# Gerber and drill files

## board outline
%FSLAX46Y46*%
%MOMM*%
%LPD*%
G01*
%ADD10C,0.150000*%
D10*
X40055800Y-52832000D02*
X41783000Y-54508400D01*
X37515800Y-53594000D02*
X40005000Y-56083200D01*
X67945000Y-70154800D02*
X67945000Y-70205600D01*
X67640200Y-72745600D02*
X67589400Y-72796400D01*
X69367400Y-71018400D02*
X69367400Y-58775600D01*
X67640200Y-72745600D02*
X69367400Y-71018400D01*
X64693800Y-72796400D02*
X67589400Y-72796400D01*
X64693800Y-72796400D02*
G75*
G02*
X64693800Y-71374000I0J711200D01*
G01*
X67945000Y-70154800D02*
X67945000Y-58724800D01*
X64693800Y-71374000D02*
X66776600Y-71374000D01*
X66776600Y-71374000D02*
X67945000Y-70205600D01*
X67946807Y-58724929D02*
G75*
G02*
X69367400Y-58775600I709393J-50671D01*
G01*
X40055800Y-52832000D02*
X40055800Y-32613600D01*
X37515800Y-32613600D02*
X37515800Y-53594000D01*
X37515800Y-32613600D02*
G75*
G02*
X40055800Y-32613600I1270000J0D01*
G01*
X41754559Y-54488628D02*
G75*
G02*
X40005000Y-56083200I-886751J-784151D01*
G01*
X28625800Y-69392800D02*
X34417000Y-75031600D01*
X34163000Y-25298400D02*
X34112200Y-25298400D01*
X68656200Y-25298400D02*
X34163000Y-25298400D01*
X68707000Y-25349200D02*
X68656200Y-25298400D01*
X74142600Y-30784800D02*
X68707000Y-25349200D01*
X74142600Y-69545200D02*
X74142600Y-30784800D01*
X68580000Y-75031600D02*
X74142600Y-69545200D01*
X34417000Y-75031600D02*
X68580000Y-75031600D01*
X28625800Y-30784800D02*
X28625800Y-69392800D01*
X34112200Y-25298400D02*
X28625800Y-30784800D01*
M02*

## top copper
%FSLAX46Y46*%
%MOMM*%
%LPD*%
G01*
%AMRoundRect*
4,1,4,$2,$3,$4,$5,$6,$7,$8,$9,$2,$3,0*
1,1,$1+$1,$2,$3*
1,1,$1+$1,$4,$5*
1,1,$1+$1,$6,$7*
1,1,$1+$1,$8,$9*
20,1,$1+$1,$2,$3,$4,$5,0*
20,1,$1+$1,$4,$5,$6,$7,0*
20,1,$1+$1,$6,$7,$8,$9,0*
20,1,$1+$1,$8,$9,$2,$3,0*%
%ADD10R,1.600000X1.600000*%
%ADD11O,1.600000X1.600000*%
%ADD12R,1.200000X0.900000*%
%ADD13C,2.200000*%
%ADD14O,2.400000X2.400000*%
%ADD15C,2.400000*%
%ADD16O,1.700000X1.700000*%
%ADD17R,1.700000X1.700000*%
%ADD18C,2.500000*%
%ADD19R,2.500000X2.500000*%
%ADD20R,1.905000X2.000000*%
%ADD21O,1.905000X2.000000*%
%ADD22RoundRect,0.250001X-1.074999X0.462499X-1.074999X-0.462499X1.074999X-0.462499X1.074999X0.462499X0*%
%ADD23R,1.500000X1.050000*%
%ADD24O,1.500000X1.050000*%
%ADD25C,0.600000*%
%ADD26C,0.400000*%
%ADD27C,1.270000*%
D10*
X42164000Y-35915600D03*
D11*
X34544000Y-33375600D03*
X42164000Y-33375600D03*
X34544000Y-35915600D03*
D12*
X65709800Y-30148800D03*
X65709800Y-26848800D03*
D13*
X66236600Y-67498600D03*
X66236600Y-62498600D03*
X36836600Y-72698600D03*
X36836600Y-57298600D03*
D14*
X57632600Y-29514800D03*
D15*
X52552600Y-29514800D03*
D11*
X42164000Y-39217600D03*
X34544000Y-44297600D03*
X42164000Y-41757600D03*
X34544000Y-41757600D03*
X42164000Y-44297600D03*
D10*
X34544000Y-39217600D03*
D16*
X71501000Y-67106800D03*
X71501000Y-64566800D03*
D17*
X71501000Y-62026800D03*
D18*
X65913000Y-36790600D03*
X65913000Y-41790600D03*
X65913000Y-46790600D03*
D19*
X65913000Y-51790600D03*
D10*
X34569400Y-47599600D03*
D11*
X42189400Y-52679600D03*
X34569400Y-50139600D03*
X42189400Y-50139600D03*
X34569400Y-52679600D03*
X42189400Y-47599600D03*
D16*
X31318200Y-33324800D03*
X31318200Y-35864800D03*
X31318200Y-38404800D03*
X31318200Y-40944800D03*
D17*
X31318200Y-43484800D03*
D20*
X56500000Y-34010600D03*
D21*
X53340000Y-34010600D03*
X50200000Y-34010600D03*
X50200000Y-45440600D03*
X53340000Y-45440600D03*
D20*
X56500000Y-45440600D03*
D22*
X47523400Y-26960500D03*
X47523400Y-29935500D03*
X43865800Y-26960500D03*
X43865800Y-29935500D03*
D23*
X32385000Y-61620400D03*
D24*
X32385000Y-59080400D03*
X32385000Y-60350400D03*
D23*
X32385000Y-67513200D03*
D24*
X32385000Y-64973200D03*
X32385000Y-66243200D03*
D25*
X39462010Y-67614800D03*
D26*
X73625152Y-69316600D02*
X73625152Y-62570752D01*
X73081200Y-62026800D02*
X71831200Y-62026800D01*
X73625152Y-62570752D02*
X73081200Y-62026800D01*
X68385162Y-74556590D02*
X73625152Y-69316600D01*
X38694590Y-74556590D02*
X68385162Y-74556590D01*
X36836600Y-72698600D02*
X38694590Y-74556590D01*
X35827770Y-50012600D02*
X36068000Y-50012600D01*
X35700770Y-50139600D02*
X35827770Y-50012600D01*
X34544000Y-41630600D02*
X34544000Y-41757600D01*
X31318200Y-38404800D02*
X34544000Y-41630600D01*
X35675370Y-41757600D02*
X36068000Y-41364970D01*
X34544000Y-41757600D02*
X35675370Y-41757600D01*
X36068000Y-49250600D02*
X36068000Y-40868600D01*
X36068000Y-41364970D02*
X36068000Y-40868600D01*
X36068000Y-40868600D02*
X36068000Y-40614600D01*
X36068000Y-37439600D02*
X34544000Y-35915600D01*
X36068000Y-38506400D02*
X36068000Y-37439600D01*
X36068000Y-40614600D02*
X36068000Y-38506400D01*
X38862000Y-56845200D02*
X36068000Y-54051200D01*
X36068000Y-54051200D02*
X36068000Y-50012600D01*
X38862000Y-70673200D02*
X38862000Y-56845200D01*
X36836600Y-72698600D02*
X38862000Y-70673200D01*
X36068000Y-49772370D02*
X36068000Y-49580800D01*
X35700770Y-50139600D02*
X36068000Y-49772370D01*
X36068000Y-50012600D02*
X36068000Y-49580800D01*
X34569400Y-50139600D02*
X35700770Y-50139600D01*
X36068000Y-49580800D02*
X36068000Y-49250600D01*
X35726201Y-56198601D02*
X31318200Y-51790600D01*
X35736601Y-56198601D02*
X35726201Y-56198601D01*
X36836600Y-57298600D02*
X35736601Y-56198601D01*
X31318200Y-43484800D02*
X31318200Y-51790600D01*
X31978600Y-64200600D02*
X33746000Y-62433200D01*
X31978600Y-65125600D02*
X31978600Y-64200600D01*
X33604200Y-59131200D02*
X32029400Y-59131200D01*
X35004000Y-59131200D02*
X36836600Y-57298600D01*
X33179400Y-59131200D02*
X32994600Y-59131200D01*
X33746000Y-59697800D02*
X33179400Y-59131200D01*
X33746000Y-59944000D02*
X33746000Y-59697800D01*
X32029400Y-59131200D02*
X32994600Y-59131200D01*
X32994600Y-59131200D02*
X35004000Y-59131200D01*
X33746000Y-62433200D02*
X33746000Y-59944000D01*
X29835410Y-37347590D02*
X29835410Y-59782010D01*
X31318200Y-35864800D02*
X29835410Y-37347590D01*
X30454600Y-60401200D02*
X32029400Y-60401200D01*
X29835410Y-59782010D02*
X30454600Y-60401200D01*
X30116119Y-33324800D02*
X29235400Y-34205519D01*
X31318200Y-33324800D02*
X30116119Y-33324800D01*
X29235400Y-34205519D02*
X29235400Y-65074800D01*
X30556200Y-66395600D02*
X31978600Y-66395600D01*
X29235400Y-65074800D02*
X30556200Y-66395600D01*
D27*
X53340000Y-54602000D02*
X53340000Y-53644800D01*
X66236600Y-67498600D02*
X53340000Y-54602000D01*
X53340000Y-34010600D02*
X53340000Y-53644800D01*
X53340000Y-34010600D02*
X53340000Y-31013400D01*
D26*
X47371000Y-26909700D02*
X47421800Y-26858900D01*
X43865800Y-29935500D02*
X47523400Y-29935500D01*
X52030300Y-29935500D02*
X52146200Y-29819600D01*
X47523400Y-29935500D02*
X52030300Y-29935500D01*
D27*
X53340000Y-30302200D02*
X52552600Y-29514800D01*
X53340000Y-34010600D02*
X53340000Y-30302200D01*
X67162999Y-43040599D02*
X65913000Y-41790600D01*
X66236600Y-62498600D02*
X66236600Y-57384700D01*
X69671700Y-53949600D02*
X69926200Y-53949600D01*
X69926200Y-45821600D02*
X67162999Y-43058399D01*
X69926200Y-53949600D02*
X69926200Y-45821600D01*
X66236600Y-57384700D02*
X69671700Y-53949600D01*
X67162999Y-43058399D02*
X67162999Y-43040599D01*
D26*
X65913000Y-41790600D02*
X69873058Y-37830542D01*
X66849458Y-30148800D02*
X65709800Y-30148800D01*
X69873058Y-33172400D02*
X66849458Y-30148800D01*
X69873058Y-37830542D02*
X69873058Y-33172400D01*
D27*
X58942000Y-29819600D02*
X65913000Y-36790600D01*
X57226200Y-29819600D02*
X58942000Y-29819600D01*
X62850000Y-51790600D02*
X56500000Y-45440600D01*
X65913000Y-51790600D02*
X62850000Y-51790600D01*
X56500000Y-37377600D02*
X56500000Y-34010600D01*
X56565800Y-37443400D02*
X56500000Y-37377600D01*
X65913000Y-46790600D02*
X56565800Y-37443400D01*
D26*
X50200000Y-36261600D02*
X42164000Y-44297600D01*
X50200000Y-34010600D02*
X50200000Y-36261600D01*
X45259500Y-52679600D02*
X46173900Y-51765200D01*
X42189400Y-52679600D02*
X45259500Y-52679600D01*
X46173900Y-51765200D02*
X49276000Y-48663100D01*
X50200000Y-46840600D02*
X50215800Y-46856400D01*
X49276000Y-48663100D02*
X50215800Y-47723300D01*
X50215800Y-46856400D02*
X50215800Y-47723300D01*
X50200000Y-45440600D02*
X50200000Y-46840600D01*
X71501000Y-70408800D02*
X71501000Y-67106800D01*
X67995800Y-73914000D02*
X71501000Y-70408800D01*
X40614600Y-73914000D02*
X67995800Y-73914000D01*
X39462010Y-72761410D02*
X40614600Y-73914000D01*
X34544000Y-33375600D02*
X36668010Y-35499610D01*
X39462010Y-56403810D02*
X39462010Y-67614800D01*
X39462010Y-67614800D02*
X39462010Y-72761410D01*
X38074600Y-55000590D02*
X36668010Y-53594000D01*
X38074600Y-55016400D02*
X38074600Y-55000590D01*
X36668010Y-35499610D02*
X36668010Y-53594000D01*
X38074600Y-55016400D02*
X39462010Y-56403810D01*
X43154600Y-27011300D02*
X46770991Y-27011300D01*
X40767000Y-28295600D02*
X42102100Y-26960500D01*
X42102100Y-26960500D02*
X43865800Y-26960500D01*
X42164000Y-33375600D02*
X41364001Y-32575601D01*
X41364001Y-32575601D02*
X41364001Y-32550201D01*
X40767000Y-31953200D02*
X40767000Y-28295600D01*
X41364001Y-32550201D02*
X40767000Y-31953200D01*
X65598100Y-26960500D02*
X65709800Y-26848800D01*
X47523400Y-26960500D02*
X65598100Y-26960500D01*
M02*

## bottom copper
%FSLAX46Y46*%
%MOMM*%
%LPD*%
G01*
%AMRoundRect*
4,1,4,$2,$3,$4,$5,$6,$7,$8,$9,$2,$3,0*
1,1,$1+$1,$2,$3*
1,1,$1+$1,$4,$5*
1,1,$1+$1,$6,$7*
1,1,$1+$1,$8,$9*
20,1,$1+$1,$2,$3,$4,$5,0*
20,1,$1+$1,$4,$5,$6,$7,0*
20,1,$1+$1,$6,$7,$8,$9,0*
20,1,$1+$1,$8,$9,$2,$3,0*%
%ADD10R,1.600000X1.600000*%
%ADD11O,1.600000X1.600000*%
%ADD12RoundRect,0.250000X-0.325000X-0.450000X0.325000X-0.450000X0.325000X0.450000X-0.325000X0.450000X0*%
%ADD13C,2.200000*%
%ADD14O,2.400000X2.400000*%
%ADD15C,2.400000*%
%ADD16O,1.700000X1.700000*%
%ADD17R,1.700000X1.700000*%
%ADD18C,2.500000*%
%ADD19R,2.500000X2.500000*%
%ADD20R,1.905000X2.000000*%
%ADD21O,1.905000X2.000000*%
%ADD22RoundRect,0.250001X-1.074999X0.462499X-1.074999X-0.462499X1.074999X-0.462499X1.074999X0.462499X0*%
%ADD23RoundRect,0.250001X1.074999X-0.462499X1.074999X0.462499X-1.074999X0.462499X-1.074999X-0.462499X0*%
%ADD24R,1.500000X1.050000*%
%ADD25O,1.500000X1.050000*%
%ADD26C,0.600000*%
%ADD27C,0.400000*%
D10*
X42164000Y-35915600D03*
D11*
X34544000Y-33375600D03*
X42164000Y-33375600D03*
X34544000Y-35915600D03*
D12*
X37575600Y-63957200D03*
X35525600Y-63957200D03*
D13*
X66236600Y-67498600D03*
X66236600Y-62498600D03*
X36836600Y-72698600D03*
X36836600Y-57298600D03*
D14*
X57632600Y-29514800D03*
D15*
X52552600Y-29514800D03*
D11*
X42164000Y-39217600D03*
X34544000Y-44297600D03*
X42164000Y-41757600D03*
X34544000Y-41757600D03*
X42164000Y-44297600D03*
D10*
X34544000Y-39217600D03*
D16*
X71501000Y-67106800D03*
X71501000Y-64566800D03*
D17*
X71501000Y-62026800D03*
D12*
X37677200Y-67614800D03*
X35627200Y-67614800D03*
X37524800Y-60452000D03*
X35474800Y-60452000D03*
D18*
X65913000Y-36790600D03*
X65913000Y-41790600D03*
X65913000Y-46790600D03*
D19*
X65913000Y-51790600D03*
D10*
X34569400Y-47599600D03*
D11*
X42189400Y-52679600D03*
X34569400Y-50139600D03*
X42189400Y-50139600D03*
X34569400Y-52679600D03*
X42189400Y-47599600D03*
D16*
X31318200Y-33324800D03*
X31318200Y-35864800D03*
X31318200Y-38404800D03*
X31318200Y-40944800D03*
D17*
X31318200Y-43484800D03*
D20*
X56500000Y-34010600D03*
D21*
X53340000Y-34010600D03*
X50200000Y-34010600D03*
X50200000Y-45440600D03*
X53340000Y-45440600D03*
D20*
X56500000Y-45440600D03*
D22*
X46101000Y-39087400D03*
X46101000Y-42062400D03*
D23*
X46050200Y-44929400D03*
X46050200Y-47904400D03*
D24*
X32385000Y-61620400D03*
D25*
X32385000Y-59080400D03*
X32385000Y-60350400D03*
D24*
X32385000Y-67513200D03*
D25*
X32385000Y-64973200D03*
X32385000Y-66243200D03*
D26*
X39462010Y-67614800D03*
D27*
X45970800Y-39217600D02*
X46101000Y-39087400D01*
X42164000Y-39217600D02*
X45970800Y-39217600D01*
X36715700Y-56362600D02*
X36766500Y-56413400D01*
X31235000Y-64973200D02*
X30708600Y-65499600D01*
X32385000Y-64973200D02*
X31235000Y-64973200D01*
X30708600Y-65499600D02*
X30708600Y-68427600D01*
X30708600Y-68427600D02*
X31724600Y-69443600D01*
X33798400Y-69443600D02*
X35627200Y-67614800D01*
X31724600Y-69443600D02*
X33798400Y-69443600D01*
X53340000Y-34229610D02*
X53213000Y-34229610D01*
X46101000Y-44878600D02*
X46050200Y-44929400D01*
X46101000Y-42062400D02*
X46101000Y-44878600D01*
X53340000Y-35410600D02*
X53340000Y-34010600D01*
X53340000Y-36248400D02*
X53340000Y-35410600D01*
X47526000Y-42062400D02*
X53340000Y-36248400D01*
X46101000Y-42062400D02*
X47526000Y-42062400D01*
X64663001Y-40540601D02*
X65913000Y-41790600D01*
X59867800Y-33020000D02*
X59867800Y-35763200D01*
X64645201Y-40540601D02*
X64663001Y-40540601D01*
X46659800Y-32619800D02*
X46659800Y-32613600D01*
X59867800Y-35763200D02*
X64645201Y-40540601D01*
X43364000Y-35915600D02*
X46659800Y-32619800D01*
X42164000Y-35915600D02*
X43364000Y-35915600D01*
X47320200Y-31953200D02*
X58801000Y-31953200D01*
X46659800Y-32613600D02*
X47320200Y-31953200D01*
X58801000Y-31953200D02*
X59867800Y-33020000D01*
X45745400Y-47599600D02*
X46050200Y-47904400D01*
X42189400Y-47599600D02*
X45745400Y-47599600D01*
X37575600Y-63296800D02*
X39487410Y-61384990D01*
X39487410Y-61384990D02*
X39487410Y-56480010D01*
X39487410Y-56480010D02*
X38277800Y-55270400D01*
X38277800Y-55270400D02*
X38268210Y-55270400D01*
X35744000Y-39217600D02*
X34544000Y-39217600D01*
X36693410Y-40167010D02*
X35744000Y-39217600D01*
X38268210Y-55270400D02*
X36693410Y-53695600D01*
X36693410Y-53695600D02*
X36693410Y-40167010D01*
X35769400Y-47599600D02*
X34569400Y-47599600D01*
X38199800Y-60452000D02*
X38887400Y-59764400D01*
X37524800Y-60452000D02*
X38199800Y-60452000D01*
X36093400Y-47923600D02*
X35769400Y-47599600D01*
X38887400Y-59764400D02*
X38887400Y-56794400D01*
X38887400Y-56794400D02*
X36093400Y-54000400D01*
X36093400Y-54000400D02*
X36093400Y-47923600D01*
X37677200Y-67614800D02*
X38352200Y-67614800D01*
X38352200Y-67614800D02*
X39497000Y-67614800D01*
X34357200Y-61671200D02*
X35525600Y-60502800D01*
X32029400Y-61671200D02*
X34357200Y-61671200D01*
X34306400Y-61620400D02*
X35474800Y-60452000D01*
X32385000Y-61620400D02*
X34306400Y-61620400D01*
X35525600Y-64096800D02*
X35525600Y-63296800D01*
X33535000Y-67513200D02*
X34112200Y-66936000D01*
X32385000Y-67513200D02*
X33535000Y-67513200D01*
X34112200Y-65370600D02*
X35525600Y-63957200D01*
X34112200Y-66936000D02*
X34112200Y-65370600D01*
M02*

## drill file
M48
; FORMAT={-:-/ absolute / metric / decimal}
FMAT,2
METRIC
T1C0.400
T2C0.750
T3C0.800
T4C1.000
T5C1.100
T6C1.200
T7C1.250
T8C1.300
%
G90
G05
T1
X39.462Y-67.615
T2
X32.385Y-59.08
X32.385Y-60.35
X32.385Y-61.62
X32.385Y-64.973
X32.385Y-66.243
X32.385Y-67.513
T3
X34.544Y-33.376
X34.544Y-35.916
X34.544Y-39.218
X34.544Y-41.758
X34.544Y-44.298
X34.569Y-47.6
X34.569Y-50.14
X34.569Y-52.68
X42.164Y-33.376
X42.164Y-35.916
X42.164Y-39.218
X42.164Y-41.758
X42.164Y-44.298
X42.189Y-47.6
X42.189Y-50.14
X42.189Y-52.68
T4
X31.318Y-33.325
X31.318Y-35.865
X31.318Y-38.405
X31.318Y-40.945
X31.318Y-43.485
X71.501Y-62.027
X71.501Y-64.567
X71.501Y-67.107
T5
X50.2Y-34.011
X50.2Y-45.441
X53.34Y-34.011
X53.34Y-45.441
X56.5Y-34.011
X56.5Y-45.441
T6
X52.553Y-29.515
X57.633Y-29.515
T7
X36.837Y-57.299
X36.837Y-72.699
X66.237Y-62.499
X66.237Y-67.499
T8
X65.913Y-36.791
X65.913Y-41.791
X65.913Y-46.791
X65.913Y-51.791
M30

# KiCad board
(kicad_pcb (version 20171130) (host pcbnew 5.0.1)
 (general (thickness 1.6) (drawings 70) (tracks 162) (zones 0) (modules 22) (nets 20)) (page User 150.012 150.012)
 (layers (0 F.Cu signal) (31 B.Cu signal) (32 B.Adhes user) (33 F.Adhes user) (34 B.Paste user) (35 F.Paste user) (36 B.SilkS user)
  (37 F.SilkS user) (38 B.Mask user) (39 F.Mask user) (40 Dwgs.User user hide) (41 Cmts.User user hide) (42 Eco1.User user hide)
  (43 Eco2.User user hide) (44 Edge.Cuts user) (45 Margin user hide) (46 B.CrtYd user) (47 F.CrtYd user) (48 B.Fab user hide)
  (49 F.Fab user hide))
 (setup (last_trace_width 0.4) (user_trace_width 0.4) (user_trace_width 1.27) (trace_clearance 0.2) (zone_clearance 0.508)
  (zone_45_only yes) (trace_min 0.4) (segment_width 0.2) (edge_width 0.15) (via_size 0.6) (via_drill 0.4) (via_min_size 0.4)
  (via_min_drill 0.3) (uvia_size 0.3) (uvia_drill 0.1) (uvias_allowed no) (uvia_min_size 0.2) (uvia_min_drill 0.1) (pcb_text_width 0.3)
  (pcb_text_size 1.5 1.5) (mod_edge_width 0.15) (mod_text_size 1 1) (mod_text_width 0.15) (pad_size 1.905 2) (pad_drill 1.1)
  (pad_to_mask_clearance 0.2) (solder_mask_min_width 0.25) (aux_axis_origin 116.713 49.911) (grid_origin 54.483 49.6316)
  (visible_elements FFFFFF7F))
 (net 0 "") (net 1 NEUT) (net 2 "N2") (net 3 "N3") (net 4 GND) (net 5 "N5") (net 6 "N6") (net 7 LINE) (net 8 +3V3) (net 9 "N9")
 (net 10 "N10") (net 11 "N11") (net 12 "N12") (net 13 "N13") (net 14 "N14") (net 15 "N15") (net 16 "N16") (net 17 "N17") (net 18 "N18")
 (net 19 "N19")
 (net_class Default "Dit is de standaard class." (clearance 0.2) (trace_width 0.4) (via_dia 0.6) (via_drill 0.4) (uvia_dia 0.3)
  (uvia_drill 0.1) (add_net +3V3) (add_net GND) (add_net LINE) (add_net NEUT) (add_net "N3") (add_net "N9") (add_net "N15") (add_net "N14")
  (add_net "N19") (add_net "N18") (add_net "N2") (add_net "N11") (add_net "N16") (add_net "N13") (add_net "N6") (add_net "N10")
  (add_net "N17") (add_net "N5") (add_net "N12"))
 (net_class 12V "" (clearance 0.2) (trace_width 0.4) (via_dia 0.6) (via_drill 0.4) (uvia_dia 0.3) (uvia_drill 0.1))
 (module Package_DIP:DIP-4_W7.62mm (layer F.Cu) (at 42.164 35.9156 180)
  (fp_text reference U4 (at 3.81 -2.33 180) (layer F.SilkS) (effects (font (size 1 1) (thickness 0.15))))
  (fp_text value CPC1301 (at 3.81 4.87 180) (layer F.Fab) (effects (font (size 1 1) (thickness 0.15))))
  (pad 1 thru_hole rect (at 0 0 180) (size 1.6 1.6) (drill 0.8) (layers *.Cu *.Mask) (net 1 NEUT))
  (pad 3 thru_hole oval (at 7.62 2.54 180) (size 1.6 1.6) (drill 0.8) (layers *.Cu *.Mask) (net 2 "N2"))
  (pad 2 thru_hole oval (at 0 2.54 180) (size 1.6 1.6) (drill 0.8) (layers *.Cu *.Mask) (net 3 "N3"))
  (pad 4 thru_hole oval (at 7.62 0 180) (size 1.6 1.6) (drill 0.8) (layers *.Cu *.Mask) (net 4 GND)))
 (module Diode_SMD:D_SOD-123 (layer F.Cu) (at 65.7098 28.4988 270)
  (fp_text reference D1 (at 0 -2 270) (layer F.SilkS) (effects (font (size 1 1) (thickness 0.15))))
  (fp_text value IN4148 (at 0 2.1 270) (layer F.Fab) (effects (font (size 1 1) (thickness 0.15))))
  (pad 2 smd rect (at 1.65 0 270) (size 0.9 1.2) (layers F.Cu F.Paste F.Mask) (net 1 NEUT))
  (pad 1 smd rect (at -1.65 0 270) (size 0.9 1.2) (layers F.Cu F.Paste F.Mask) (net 3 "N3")))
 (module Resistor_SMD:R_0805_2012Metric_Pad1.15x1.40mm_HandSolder (layer B.Cu) (at 36.5506 63.9572)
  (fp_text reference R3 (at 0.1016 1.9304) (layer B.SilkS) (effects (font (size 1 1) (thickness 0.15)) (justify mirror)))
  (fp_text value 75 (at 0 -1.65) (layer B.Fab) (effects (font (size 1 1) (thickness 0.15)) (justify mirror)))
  (pad 2 smd roundrect (at 1.025 0) (size 1.15 1.4) (layers B.Cu B.Paste B.Mask) (roundrect_rratio 0.217391) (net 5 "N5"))
  (pad 1 smd roundrect (at -1.025 0) (size 1.15 1.4) (layers B.Cu B.Paste B.Mask) (roundrect_rratio 0.217391) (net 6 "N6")))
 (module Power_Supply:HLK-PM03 (layer F.Cu) (at 51.5366 64.9986 180)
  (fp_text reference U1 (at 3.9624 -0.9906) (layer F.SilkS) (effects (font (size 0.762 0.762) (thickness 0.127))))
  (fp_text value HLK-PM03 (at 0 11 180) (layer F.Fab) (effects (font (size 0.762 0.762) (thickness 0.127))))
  (pad 1 thru_hole circle (at -14.7 -2.5 180) (size 2.2 2.2) (drill 1.25) (layers *.Cu *.Mask) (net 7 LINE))
  (pad 2 thru_hole circle (at -14.7 2.5 180) (size 2.2 2.2) (drill 1.25) (layers *.Cu *.Mask) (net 1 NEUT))
  (pad 3 thru_hole circle (at 14.7 -7.7 180) (size 2.2 2.2) (drill 1.25) (layers *.Cu *.Mask) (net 4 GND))
  (pad 4 thru_hole circle (at 14.7 7.7 180) (size 2.2 2.2) (drill 1.25) (layers *.Cu *.Mask) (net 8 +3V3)))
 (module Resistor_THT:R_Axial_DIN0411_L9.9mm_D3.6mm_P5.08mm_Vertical (layer F.Cu) (at 52.5526 29.5148)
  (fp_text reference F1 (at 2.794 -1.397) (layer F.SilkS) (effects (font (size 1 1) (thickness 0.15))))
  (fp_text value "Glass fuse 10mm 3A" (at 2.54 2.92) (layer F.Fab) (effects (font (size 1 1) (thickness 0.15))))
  (pad 2 thru_hole oval (at 5.08 0) (size 2.4 2.4) (drill 1.2) (layers *.Cu *.Mask) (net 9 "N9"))
  (pad 1 thru_hole circle (at 0 0) (size 2.4 2.4) (drill 1.2) (layers *.Cu *.Mask) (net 7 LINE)))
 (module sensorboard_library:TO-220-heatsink (layer F.Cu) (at 53.3146 37.9476)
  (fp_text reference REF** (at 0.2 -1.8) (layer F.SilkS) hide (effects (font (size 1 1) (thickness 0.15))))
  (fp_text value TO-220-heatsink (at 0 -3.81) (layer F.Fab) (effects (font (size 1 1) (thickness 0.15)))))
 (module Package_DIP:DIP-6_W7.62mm (layer F.Cu) (at 34.544 39.2176)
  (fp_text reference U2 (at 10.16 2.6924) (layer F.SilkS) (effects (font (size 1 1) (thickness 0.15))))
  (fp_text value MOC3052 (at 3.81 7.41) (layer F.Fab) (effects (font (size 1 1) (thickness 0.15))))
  (pad 6 thru_hole oval (at 7.62 0) (size 1.6 1.6) (drill 0.8) (layers *.Cu *.Mask) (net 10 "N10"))
  (pad 3 thru_hole oval (at 0 5.08) (size 1.6 1.6) (drill 0.8) (layers *.Cu *.Mask))
  (pad 5 thru_hole oval (at 7.62 2.54) (size 1.6 1.6) (drill 0.8) (layers *.Cu *.Mask))
  (pad 2 thru_hole oval (at 0 2.54) (size 1.6 1.6) (drill 0.8) (layers *.Cu *.Mask) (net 4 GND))
  (pad 4 thru_hole oval (at 7.62 5.08) (size 1.6 1.6) (drill 0.8) (layers *.Cu *.Mask) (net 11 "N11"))
  (pad 1 thru_hole rect (at 0 0) (size 1.6 1.6) (drill 0.8) (layers *.Cu *.Mask) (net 5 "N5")))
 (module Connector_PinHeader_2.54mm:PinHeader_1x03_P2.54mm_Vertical (layer B.Cu) (at 71.501 62.0268 180)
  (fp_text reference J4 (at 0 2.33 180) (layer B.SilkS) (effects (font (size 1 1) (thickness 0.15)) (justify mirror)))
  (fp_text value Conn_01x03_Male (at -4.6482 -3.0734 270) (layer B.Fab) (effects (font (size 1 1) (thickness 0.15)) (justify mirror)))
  (pad 3 thru_hole oval (at 0 -5.08 180) (size 1.7 1.7) (drill 1) (layers *.Cu *.Mask) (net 2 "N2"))
  (pad 2 thru_hole oval (at 0 -2.54 180) (size 1.7 1.7) (drill 1) (layers *.Cu *.Mask))
  (pad 1 thru_hole rect (at 0 0 180) (size 1.7 1.7) (drill 1) (layers *.Cu *.Mask) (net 4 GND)))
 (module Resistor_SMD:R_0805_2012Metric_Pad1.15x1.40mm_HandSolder (layer B.Cu) (at 36.6522 67.6148)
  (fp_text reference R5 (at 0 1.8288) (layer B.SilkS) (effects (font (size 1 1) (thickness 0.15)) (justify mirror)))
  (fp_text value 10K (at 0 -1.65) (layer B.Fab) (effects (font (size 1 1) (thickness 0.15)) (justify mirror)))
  (pad 2 smd roundrect (at 1.025 0) (size 1.15 1.4) (layers B.Cu B.Paste B.Mask) (roundrect_rratio 0.217391) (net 2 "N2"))
  (pad 1 smd roundrect (at -1.025 0) (size 1.15 1.4) (layers B.Cu B.Paste B.Mask) (roundrect_rratio 0.217391) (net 8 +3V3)))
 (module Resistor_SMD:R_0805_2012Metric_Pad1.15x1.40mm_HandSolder (layer B.Cu) (at 36.4998 60.452)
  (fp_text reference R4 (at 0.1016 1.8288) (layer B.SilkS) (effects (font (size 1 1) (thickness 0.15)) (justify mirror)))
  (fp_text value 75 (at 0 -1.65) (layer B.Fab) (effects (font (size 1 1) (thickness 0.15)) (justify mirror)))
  (pad 2 smd roundrect (at 1.025 0) (size 1.15 1.4) (layers B.Cu B.Paste B.Mask) (roundrect_rratio 0.217391) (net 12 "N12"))
  (pad 1 smd roundrect (at -1.025 0) (size 1.15 1.4) (layers B.Cu B.Paste B.Mask) (roundrect_rratio 0.217391) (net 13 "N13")))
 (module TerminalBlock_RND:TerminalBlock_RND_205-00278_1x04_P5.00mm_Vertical (layer F.Cu) (at 65.913 51.7906 90)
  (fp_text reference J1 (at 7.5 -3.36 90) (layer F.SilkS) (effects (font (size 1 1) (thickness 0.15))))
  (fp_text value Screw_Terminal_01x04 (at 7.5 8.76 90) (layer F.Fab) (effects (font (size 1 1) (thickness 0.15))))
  (pad 4 thru_hole circle (at 15 0 90) (size 2.5 2.5) (drill 1.3) (layers *.Cu *.Mask) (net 9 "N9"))
  (pad 3 thru_hole circle (at 10 0 90) (size 2.5 2.5) (drill 1.3) (layers *.Cu *.Mask) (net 1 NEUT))
  (pad 2 thru_hole circle (at 5 0 90) (size 2.5 2.5) (drill 1.3) (layers *.Cu *.Mask) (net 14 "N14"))
  (pad 1 thru_hole rect (at 0 0 90) (size 2.5 2.5) (drill 1.3) (layers *.Cu *.Mask) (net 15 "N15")))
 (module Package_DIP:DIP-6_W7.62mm (layer F.Cu) (at 34.5694 47.5996)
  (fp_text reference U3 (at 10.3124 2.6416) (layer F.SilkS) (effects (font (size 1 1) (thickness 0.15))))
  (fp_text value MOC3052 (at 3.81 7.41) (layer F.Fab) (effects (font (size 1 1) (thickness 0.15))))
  (pad 1 thru_hole rect (at 0 0) (size 1.6 1.6) (drill 0.8) (layers *.Cu *.Mask) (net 12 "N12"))
  (pad 4 thru_hole oval (at 7.62 5.08) (size 1.6 1.6) (drill 0.8) (layers *.Cu *.Mask) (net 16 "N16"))
  (pad 2 thru_hole oval (at 0 2.54) (size 1.6 1.6) (drill 0.8) (layers *.Cu *.Mask) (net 4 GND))
  (pad 5 thru_hole oval (at 7.62 2.54) (size 1.6 1.6) (drill 0.8) (layers *.Cu *.Mask))
  (pad 3 thru_hole oval (at 0 5.08) (size 1.6 1.6) (drill 0.8) (layers *.Cu *.Mask))
  (pad 6 thru_hole oval (at 7.62 0) (size 1.6 1.6) (drill 0.8) (layers *.Cu *.Mask) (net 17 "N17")))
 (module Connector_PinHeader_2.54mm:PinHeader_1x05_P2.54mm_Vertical (layer B.Cu) (at 31.3182 43.4848)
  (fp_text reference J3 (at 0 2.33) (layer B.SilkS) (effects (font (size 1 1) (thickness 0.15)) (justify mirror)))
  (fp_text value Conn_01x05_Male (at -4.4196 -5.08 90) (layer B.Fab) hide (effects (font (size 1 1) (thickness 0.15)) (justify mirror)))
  (pad 5 thru_hole oval (at 0 -10.16) (size 1.7 1.7) (drill 1) (layers *.Cu *.Mask) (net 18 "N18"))
  (pad 4 thru_hole oval (at 0 -7.62) (size 1.7 1.7) (drill 1) (layers *.Cu *.Mask) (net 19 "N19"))
  (pad 3 thru_hole oval (at 0 -5.08) (size 1.7 1.7) (drill 1) (layers *.Cu *.Mask) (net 4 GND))
  (pad 2 thru_hole oval (at 0 -2.54) (size 1.7 1.7) (drill 1) (layers *.Cu *.Mask))
  (pad 1 thru_hole rect (at 0 0) (size 1.7 1.7) (drill 1) (layers *.Cu *.Mask) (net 8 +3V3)))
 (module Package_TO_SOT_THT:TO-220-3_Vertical (layer F.Cu) (at 55.88 34.0106 180)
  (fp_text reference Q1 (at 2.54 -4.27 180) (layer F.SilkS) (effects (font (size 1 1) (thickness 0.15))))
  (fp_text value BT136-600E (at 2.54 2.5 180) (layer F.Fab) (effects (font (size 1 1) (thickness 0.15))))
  (pad 1 thru_hole rect (at -0.62 0 180) (size 1.905 2) (drill 1.1) (layers *.Cu *.Mask) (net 14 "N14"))
  (pad 2 thru_hole oval (at 2.54 0 180) (size 1.905 2) (drill 1.1) (layers *.Cu *.Mask) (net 7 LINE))
  (pad 3 thru_hole oval (at 5.68 0 180) (size 1.905 2) (drill 1.1) (layers *.Cu *.Mask) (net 11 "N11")))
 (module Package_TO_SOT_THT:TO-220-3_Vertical (layer F.Cu) (at 55.88 45.4406 180)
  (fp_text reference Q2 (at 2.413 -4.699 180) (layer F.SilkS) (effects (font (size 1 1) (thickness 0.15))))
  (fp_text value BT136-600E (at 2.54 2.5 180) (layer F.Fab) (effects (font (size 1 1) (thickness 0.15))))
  (pad 3 thru_hole oval (at 5.68 0 180) (size 1.905 2) (drill 1.1) (layers *.Cu *.Mask) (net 16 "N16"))
  (pad 2 thru_hole oval (at 2.54 0 180) (size 1.905 2) (drill 1.1) (layers *.Cu *.Mask) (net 7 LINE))
  (pad 1 thru_hole rect (at -0.62 0 180) (size 1.905 2) (drill 1.1) (layers *.Cu *.Mask) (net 15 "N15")))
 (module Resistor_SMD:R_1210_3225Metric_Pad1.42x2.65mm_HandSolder (layer B.Cu) (at 46.101 40.5749 270)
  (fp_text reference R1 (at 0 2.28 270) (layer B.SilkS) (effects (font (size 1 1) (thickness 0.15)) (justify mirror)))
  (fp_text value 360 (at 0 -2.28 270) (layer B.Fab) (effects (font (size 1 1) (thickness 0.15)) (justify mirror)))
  (pad 1 smd roundrect (at -1.4875 0 270) (size 1.425 2.65) (layers B.Cu B.Paste B.Mask) (roundrect_rratio 0.175439) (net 10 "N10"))
  (pad 2 smd roundrect (at 1.4875 0 270) (size 1.425 2.65) (layers B.Cu B.Paste B.Mask) (roundrect_rratio 0.175439) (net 7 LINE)))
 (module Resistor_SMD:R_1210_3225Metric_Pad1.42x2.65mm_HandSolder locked (layer B.Cu) (at 46.0502 46.4169 90)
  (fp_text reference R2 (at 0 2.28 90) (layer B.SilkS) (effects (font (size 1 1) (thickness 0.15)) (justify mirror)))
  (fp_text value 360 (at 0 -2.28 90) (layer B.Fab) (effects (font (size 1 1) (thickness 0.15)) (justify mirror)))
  (pad 2 smd roundrect (at 1.4875 0 90) (size 1.425 2.65) (layers B.Cu B.Paste B.Mask) (roundrect_rratio 0.175439) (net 7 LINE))
  (pad 1 smd roundrect (at -1.4875 0 90) (size 1.425 2.65) (layers B.Cu B.Paste B.Mask) (roundrect_rratio 0.175439) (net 17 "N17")))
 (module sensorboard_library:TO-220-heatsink (layer F.Cu) (at 53.1114 49.4792)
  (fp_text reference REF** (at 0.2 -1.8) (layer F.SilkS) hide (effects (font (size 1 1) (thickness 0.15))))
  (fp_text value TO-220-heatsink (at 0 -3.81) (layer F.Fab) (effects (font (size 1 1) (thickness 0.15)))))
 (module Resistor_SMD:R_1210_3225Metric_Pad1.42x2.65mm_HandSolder (layer F.Cu) (at 47.5234 28.448 270)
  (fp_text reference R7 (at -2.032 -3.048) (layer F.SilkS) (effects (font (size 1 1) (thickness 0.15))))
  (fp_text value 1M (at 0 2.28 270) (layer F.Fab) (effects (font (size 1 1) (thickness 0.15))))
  (pad 1 smd roundrect (at -1.4875 0 270) (size 1.425 2.65) (layers F.Cu F.Paste F.Mask) (roundrect_rratio 0.175439) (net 3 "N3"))
  (pad 2 smd roundrect (at 1.4875 0 270) (size 1.425 2.65) (layers F.Cu F.Paste F.Mask) (roundrect_rratio 0.175439) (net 7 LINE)))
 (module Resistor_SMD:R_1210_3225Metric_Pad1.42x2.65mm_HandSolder (layer F.Cu) (at 43.8658 28.448 270)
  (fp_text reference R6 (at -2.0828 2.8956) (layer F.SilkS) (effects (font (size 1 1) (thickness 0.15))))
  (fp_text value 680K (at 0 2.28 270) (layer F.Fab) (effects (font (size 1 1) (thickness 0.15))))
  (pad 1 smd roundrect (at -1.4875 0 270) (size 1.425 2.65) (layers F.Cu F.Paste F.Mask) (roundrect_rratio 0.175439) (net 3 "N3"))
  (pad 2 smd roundrect (at 1.4875 0 270) (size 1.425 2.65) (layers F.Cu F.Paste F.Mask) (roundrect_rratio 0.175439) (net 7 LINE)))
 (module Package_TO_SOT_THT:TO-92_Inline (layer F.Cu) (at 32.385 61.6204 90)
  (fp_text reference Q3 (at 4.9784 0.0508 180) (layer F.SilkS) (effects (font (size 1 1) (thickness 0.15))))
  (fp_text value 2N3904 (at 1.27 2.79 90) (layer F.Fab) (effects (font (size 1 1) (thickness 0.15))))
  (pad 1 thru_hole rect (at 0 0 90) (size 1.05 1.5) (drill 0.75) (layers *.Cu *.Mask) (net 13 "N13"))
  (pad 3 thru_hole oval (at 2.54 0 90) (size 1.05 1.5) (drill 0.75) (layers *.Cu *.Mask) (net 8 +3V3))
  (pad 2 thru_hole oval (at 1.27 0 90) (size 1.05 1.5) (drill 0.75) (layers *.Cu *.Mask) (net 19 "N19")))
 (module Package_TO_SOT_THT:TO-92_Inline (layer F.Cu) (at 32.385 67.5132 90)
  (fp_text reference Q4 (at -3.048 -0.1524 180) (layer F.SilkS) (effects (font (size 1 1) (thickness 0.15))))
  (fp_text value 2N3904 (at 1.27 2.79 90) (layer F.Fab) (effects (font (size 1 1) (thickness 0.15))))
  (pad 1 thru_hole rect (at 0 0 90) (size 1.05 1.5) (drill 0.75) (layers *.Cu *.Mask) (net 6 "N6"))
  (pad 3 thru_hole oval (at 2.54 0 90) (size 1.05 1.5) (drill 0.75) (layers *.Cu *.Mask) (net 8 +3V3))
  (pad 2 thru_hole oval (at 1.27 0 90) (size 1.05 1.5) (drill 0.75) (layers *.Cu *.Mask) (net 18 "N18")))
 (gr_line (start 40.0558 52.832) (end 41.783 54.5084) (layer Edge.Cuts) (width 0.15))
 (gr_line (start 37.5158 53.594) (end 40.005 56.0832) (layer Edge.Cuts) (width 0.15))
 (gr_line (start 67.945 70.1548) (end 67.945 70.2056) (layer Edge.Cuts) (width 0.15))
 (gr_line (start 67.6402 72.7456) (end 67.5894 72.7964) (layer Edge.Cuts) (width 0.15))
 (gr_line (start 69.3674 71.0184) (end 69.3674 58.7756) (layer Edge.Cuts) (width 0.15))
 (gr_line (start 67.6402 72.7456) (end 69.3674 71.0184) (layer Edge.Cuts) (width 0.15))
 (gr_line (start 64.6938 72.7964) (end 67.5894 72.7964) (layer Edge.Cuts) (width 0.15))
 (gr_arc (start 64.6938 72.0852) (end 64.6938 71.374) (angle -180) (layer Edge.Cuts) (width 0.15))
 (gr_line (start 67.945 70.1548) (end 67.945 58.7248) (layer Edge.Cuts) (width 0.15))
 (gr_line (start 64.6938 71.374) (end 66.7766 71.374) (layer Edge.Cuts) (width 0.15))
 (gr_line (start 66.7766 71.374) (end 67.945 70.2056) (layer Edge.Cuts) (width 0.15))
 (gr_arc (start 68.6562 58.7756) (end 69.3674 58.7756) (angle -175.9143832) (layer Edge.Cuts) (width 0.15))
 (gr_line (start 40.0558 52.832) (end 40.0558 32.6136) (layer Edge.Cuts) (width 0.15))
 (gr_line (start 37.5158 32.6136) (end 37.5158 53.594) (layer Edge.Cuts) (width 0.15))
 (gr_arc (start 38.7858 32.6136) (end 40.0558 32.6136) (angle -180) (layer Edge.Cuts) (width 0.15))
 (gr_arc (start 40.867808 55.272779) (end 40.005 56.0832) (angle -178.279507) (layer Edge.Cuts) (width 0.15))
 (gr_line (start 28.6258 69.3928) (end 34.417 75.0316) (layer Edge.Cuts) (width 0.15))
 (gr_line (start 34.163 25.2984) (end 34.1122 25.2984) (layer Edge.Cuts) (width 0.15))
 (gr_line (start 68.6562 25.2984) (end 34.163 25.2984) (layer Edge.Cuts) (width 0.15))
 (gr_line (start 68.707 25.3492) (end 68.6562 25.2984) (layer Edge.Cuts) (width 0.15))
 (gr_line (start 74.1426 30.7848) (end 68.707 25.3492) (layer Edge.Cuts) (width 0.15))
 (gr_line (start 74.1426 69.5452) (end 74.1426 30.7848) (layer Edge.Cuts) (width 0.15))
 (gr_line (start 68.58 75.0316) (end 74.1426 69.5452) (layer Edge.Cuts) (width 0.15))
 (gr_line (start 34.417 75.0316) (end 68.58 75.0316) (layer Edge.Cuts) (width 0.15))
 (gr_line (start 28.6258 30.7848) (end 28.6258 69.3928) (layer Edge.Cuts) (width 0.15))
 (gr_line (start 34.1122 25.2984) (end 28.6258 30.7848) (layer Edge.Cuts) (width 0.15))
 (segment (start 73.625152 69.3166) (end 73.625152 62.570752) (width 0.4) (layer F.Cu) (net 4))
 (segment (start 73.0812 62.0268) (end 71.8312 62.0268) (width 0.4) (layer F.Cu) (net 4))
 (segment (start 73.625152 62.570752) (end 73.0812 62.0268) (width 0.4) (layer F.Cu) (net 4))
 (segment (start 68.385162 74.55659) (end 73.625152 69.3166) (width 0.4) (layer F.Cu) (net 4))
 (segment (start 38.69459 74.55659) (end 68.385162 74.55659) (width 0.4) (layer F.Cu) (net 4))
 (segment (start 36.8366 72.6986) (end 38.69459 74.55659) (width 0.4) (layer F.Cu) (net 4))
 (segment (start 35.82777 50.0126) (end 36.068 50.0126) (width 0.4) (layer F.Cu) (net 4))
 (segment (start 35.70077 50.1396) (end 35.82777 50.0126) (width 0.4) (layer F.Cu) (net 4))
 (segment (start 34.544 41.6306) (end 34.544 41.7576) (width 0.4) (layer F.Cu) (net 4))
 (segment (start 31.3182 38.4048) (end 34.544 41.6306) (width 0.4) (layer F.Cu) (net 4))
 (segment (start 35.67537 41.7576) (end 36.068 41.36497) (width 0.4) (layer F.Cu) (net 4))
 (segment (start 34.544 41.7576) (end 35.67537 41.7576) (width 0.4) (layer F.Cu) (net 4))
 (segment (start 36.068 49.2506) (end 36.068 40.8686) (width 0.4) (layer F.Cu) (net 4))
 (segment (start 36.068 41.36497) (end 36.068 40.8686) (width 0.4) (layer F.Cu) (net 4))
 (segment (start 36.068 40.8686) (end 36.068 40.6146) (width 0.4) (layer F.Cu) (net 4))
 (segment (start 36.068 37.4396) (end 34.544 35.9156) (width 0.4) (layer F.Cu) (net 4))
 (segment (start 36.068 38.5064) (end 36.068 37.4396) (width 0.4) (layer F.Cu) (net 4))
 (segment (start 36.068 40.6146) (end 36.068 38.5064) (width 0.4) (layer F.Cu) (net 4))
 (segment (start 38.862 56.8452) (end 36.068 54.0512) (width 0.4) (layer F.Cu) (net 4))
 (segment (start 36.068 54.0512) (end 36.068 50.0126) (width 0.4) (layer F.Cu) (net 4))
 (segment (start 38.862 70.6732) (end 38.862 56.8452) (width 0.4) (layer F.Cu) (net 4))
 (segment (start 36.8366 72.6986) (end 38.862 70.6732) (width 0.4) (layer F.Cu) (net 4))
 (segment (start 36.068 49.77237) (end 36.068 49.5808) (width 0.4) (layer F.Cu) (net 4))
 (segment (start 35.70077 50.1396) (end 36.068 49.77237) (width 0.4) (layer F.Cu) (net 4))
 (segment (start 36.068 50.0126) (end 36.068 49.5808) (width 0.4) (layer F.Cu) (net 4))
 (segment (start 34.5694 50.1396) (end 35.70077 50.1396) (width 0.4) (layer F.Cu) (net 4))
 (segment (start 36.068 49.5808) (end 36.068 49.2506) (width 0.4) (layer F.Cu) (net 4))
 (segment (start 45.9708 39.2176) (end 46.101 39.0874) (width 0.4) (layer B.Cu) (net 10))
 (segment (start 42.164 39.2176) (end 45.9708 39.2176) (width 0.4) (layer B.Cu) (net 10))
 (segment (start 36.7157 56.3626) (end 36.7665 56.4134) (width 0.4) (layer B.Cu) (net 8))
 (segment (start 35.726201 56.198601) (end 31.3182 51.7906) (width 0.4) (layer F.Cu) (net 8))
 (segment (start 35.736601 56.198601) (end 35.726201 56.198601) (width 0.4) (layer F.Cu) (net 8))
 (segment (start 36.8366 57.2986) (end 35.736601 56.198601) (width 0.4) (layer F.Cu) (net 8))
 (segment (start 31.3182 43.4848) (end 31.3182 51.7906) (width 0.4) (layer F.Cu) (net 8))
 (segment (start 31.9786 64.2006) (end 33.746 62.4332) (width 0.4) (layer F.Cu) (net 8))
 (segment (start 31.9786 65.1256) (end 31.9786 64.2006) (width 0.4) (layer F.Cu) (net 8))
 (segment (start 33.6042 59.1312) (end 32.0294 59.1312) (width 0.4) (layer F.Cu) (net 8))
 (segment (start 35.004 59.1312) (end 36.8366 57.2986) (width 0.4) (layer F.Cu) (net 8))
 (segment (start 33.1794 59.1312) (end 32.9946 59.1312) (width 0.4) (layer F.Cu) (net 8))
 (segment (start 33.746 59.6978) (end 33.1794 59.1312) (width 0.4) (layer F.Cu) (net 8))
 (segment (start 33.746 59.944) (end 33.746 59.6978) (width 0.4) (layer F.Cu) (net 8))
 (segment (start 32.0294 59.1312) (end 32.9946 59.1312) (width 0.4) (layer F.Cu) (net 8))
 (segment (start 32.9946 59.1312) (end 35.004 59.1312) (width 0.4) (layer F.Cu) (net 8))
 (segment (start 33.746 62.4332) (end 33.746 59.944) (width 0.4) (layer F.Cu) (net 8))
 (segment (start 31.235 64.9732) (end 30.7086 65.4996) (width 0.4) (layer B.Cu) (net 8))
 (segment (start 32.385 64.9732) (end 31.235 64.9732) (width 0.4) (layer B.Cu) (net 8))
 (segment (start 30.7086 65.4996) (end 30.7086 68.4276) (width 0.4) (layer B.Cu) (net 8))
 (segment (start 30.7086 68.4276) (end 31.7246 69.4436) (width 0.4) (layer B.Cu) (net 8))
 (segment (start 33.7984 69.4436) (end 35.6272 67.6148) (width 0.4) (layer B.Cu) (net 8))
 (segment (start 31.7246 69.4436) (end 33.7984 69.4436) (width 0.4) (layer B.Cu) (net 8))
 (segment (start 29.83541 37.34759) (end 29.83541 59.78201) (width 0.4) (layer F.Cu) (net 19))
 (segment (start 31.3182 35.8648) (end 29.83541 37.34759) (width 0.4) (layer F.Cu) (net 19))
 (segment (start 30.4546 60.4012) (end 32.0294 60.4012) (width 0.4) (layer F.Cu) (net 19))
 (segment (start 29.83541 59.78201) (end 30.4546 60.4012) (width 0.4) (layer F.Cu) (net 19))
 (segment (start 30.116119 33.3248) (end 29.2354 34.205519) (width 0.4) (layer F.Cu) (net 18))
 (segment (start 31.3182 33.3248) (end 30.116119 33.3248) (width 0.4) (layer F.Cu) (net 18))
 (segment (start 29.2354 34.205519) (end 29.2354 65.0748) (width 0.4) (layer F.Cu) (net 18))
 (segment (start 30.5562 66.3956) (end 31.9786 66.3956) (width 0.4) (layer F.Cu) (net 18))
 (segment (start 29.2354 65.0748) (end 30.5562 66.3956) (width 0.4) (layer F.Cu) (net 18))
 (segment (start 53.34 34.22961) (end 53.213 34.22961) (width 0.4) (layer B.Cu) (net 7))
 (segment (start 53.34 54.602) (end 53.34 53.6448) (width 1.27) (layer F.Cu) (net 7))
 (segment (start 66.2366 67.4986) (end 53.34 54.602) (width 1.27) (layer F.Cu) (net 7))
 (segment (start 53.34 34.0106) (end 53.34 53.6448) (width 1.27) (layer F.Cu) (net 7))
 (segment (start 46.101 44.8786) (end 46.0502 44.9294) (width 0.4) (layer B.Cu) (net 7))
 (segment (start 46.101 42.0624) (end 46.101 44.8786) (width 0.4) (layer B.Cu) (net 7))
 (segment (start 53.34 35.4106) (end 53.34 34.0106) (width 0.4) (layer B.Cu) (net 7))
 (segment (start 53.34 36.2484) (end 53.34 35.4106) (width 0.4) (layer B.Cu) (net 7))
 (segment (start 47.526 42.0624) (end 53.34 36.2484) (width 0.4) (layer B.Cu) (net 7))
 (segment (start 46.101 42.0624) (end 47.526 42.0624) (width 0.4) (layer B.Cu) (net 7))
 (segment (start 53.34 34.0106) (end 53.34 31.0134) (width 1.27) (layer F.Cu) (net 7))
 (segment (start 47.371 26.9097) (end 47.4218 26.8589) (width 0.4) (layer F.Cu) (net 3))
 (segment (start 43.8658 29.9355) (end 47.5234 29.9355) (width 0.4) (layer F.Cu) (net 7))
 (segment (start 52.0303 29.9355) (end 52.1462 29.8196) (width 0.4) (layer F.Cu) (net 7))
 (segment (start 47.5234 29.9355) (end 52.0303 29.9355) (width 0.4) (layer F.Cu) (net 7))
 (segment (start 53.34 30.3022) (end 52.5526 29.5148) (width 1.27) (layer F.Cu) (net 7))
 (segment (start 53.34 34.0106) (end 53.34 30.3022) (width 1.27) (layer F.Cu) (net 7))
 (segment (start 67.162999 43.040599) (end 65.913 41.7906) (width 1.27) (layer F.Cu) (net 1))
 (segment (start 66.2366 62.4986) (end 66.2366 57.3847) (width 1.27) (layer F.Cu) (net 1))
 (segment (start 69.6717 53.9496) (end 69.9262 53.9496) (width 1.27) (layer F.Cu) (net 1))
 (segment (start 69.9262 45.8216) (end 67.162999 43.058399) (width 1.27) (layer F.Cu) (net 1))
 (segment (start 69.9262 53.9496) (end 69.9262 45.8216) (width 1.27) (layer F.Cu) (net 1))
 (segment (start 66.2366 57.3847) (end 69.6717 53.9496) (width 1.27) (layer F.Cu) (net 1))
 (segment (start 67.162999 43.058399) (end 67.162999 43.040599) (width 1.27) (layer F.Cu) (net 1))
 (segment (start 64.663001 40.540601) (end 65.913 41.7906) (width 0.4) (layer B.Cu) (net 1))
 (segment (start 59.8678 33.02) (end 59.8678 35.7632) (width 0.4) (layer B.Cu) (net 1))
 (segment (start 64.645201 40.540601) (end 64.663001 40.540601) (width 0.4) (layer B.Cu) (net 1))
 (segment (start 46.6598 32.6198) (end 46.6598 32.6136) (width 0.4) (layer B.Cu) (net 1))
 (segment (start 59.8678 35.7632) (end 64.645201 40.540601) (width 0.4) (layer B.Cu) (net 1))
 (segment (start 43.364 35.9156) (end 46.6598 32.6198) (width 0.4) (layer B.Cu) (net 1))
 (segment (start 42.164 35.9156) (end 43.364 35.9156) (width 0.4) (layer B.Cu) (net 1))
 (segment (start 47.3202 31.9532) (end 58.801 31.9532) (width 0.4) (layer B.Cu) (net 1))
 (segment (start 46.6598 32.6136) (end 47.3202 31.9532) (width 0.4) (layer B.Cu) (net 1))
 (segment (start 58.801 31.9532) (end 59.8678 33.02) (width 0.4) (layer B.Cu) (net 1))
 (segment (start 65.913 41.7906) (end 69.873058 37.830542) (width 0.4) (layer F.Cu) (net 1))
 (segment (start 66.849458 30.1488) (end 65.7098 30.1488) (width 0.4) (layer F.Cu) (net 1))
 (segment (start 69.873058 33.1724) (end 66.849458 30.1488) (width 0.4) (layer F.Cu) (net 1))
 (segment (start 69.873058 37.830542) (end 69.873058 33.1724) (width 0.4) (layer F.Cu) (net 1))
 (segment (start 58.942 29.8196) (end 65.913 36.7906) (width 1.27) (layer F.Cu) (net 9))
 (segment (start 57.2262 29.8196) (end 58.942 29.8196) (width 1.27) (layer F.Cu) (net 9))
 (segment (start 62.85 51.7906) (end 56.5 45.4406) (width 1.27) (layer F.Cu) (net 15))
 (segment (start 65.913 51.7906) (end 62.85 51.7906) (width 1.27) (layer F.Cu) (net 15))
 (segment (start 56.5 37.3776) (end 56.5 34.0106) (width 1.27) (layer F.Cu) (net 14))
 (segment (start 56.5658 37.4434) (end 56.5 37.3776) (width 1.27) (layer F.Cu) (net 14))
 (segment (start 65.913 46.7906) (end 56.5658 37.4434) (width 1.27) (layer F.Cu) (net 14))
 (segment (start 50.2 36.2616) (end 42.164 44.2976) (width 0.4) (layer F.Cu) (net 11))
 (segment (start 50.2 34.0106) (end 50.2 36.2616) (width 0.4) (layer F.Cu) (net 11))
 (segment (start 45.2595 52.6796) (end 46.1739 51.7652) (width 0.4) (layer F.Cu) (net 16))
 (segment (start 42.1894 52.6796) (end 45.2595 52.6796) (width 0.4) (layer F.Cu) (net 16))
 (segment (start 46.1739 51.7652) (end 49.276 48.6631) (width 0.4) (layer F.Cu) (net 16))
 (segment (start 50.2 46.8406) (end 50.2158 46.8564) (width 0.4) (layer F.Cu) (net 16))
 (segment (start 49.276 48.6631) (end 50.2158 47.7233) (width 0.4) (layer F.Cu) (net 16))
 (segment (start 50.2158 46.8564) (end 50.2158 47.7233) (width 0.4) (layer F.Cu) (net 16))
 (segment (start 50.2 45.4406) (end 50.2 46.8406) (width 0.4) (layer F.Cu) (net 16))
 (segment (start 45.7454 47.5996) (end 46.0502 47.9044) (width 0.4) (layer B.Cu) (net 17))
 (segment (start 42.1894 47.5996) (end 45.7454 47.5996) (width 0.4) (layer B.Cu) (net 17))
 (segment (start 37.5756 63.2968) (end 39.48741 61.38499) (width 0.4) (layer B.Cu) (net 5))
 (segment (start 39.48741 61.38499) (end 39.48741 56.48001) (width 0.4) (layer B.Cu) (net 5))
 (segment (start 39.48741 56.48001) (end 38.2778 55.2704) (width 0.4) (layer B.Cu) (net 5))
 (segment (start 38.2778 55.2704) (end 38.26821 55.2704) (width 0.4) (layer B.Cu) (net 5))
 (segment (start 35.744 39.2176) (end 34.544 39.2176) (width 0.4) (layer B.Cu) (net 5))
 (segment (start 36.69341 40.16701) (end 35.744 39.2176) (width 0.4) (layer B.Cu) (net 5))
 (segment (start 38.26821 55.2704) (end 36.69341 53.6956) (width 0.4) (layer B.Cu) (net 5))
 (segment (start 36.69341 53.6956) (end 36.69341 40.16701) (width 0.4) (layer B.Cu) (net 5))
 (segment (start 35.7694 47.5996) (end 34.5694 47.5996) (width 0.4) (layer B.Cu) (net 12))
 (segment (start 38.1998 60.452) (end 38.8874 59.7644) (width 0.4) (layer B.Cu) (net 12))
 (segment (start 37.5248 60.452) (end 38.1998 60.452) (width 0.4) (layer B.Cu) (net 12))
 (segment (start 36.0934 47.9236) (end 35.7694 47.5996) (width 0.4) (layer B.Cu) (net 12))
 (segment (start 38.8874 59.7644) (end 38.8874 56.7944) (width 0.4) (layer B.Cu) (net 12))
 (segment (start 38.8874 56.7944) (end 36.0934 54.0004) (width 0.4) (layer B.Cu) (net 12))
 (segment (start 36.0934 54.0004) (end 36.0934 47.9236) (width 0.4) (layer B.Cu) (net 12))
 (segment (start 71.501 70.4088) (end 71.501 67.1068) (width 0.4) (layer F.Cu) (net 2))
 (segment (start 67.9958 73.914) (end 71.501 70.4088) (width 0.4) (layer F.Cu) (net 2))
 (segment (start 40.6146 73.914) (end 67.9958 73.914) (width 0.4) (layer F.Cu) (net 2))
 (segment (start 39.46201 72.76141) (end 40.6146 73.914) (width 0.4) (layer F.Cu) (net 2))
 (segment (start 34.544 33.3756) (end 36.66801 35.49961) (width 0.4) (layer F.Cu) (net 2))
 (segment (start 39.46201 56.40381) (end 39.46201 67.6148) (width 0.4) (layer F.Cu) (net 2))
 (segment (start 37.6772 67.6148) (end 38.3522 67.6148) (width 0.4) (layer B.Cu) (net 2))
 (segment (start 38.3522 67.6148) (end 39.497 67.6148) (width 0.4) (layer B.Cu) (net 2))
 (segment (start 39.46201 67.6148) (end 39.46201 72.76141) (width 0.4) (layer F.Cu) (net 2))
 (via (at 39.46201 67.6148) (size 0.6) (drill 0.4) (layers F.Cu B.Cu) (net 2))
 (segment (start 38.0746 55.00059) (end 36.66801 53.594) (width 0.4) (layer F.Cu) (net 2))
 (segment (start 38.0746 55.0164) (end 38.0746 55.00059) (width 0.4) (layer F.Cu) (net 2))
 (segment (start 36.66801 35.49961) (end 36.66801 53.594) (width 0.4) (layer F.Cu) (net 2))
 (segment (start 38.0746 55.0164) (end 39.46201 56.40381) (width 0.4) (layer F.Cu) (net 2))
 (segment (start 43.1546 27.0113) (end 46.770991 27.0113) (width 0.4) (layer F.Cu) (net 3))
 (segment (start 40.767 28.2956) (end 42.1021 26.9605) (width 0.4) (layer F.Cu) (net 3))
 (segment (start 42.1021 26.9605) (end 43.8658 26.9605) (width 0.4) (layer F.Cu) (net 3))
 (segment (start 42.164 33.3756) (end 41.364001 32.575601) (width 0.4) (layer F.Cu) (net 3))
 (segment (start 41.364001 32.575601) (end 41.364001 32.550201) (width 0.4) (layer F.Cu) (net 3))
 (segment (start 40.767 31.9532) (end 40.767 28.2956) (width 0.4) (layer F.Cu) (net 3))
 (segment (start 41.364001 32.550201) (end 40.767 31.9532) (width 0.4) (layer F.Cu) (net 3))
 (segment (start 65.5981 26.9605) (end 65.7098 26.8488) (width 0.4) (layer F.Cu) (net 3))
 (segment (start 47.5234 26.9605) (end 65.5981 26.9605) (width 0.4) (layer F.Cu) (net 3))
 (segment (start 34.3572 61.6712) (end 35.5256 60.5028) (width 0.4) (layer B.Cu) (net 13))
 (segment (start 32.0294 61.6712) (end 34.3572 61.6712) (width 0.4) (layer B.Cu) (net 13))
 (segment (start 34.3064 61.6204) (end 35.4748 60.452) (width 0.4) (layer B.Cu) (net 13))
 (segment (start 32.385 61.6204) (end 34.3064 61.6204) (width 0.4) (layer B.Cu) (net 13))
 (segment (start 35.5256 64.0968) (end 35.5256 63.2968) (width 0.4) (layer B.Cu) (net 6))
 (segment (start 33.535 67.5132) (end 34.1122 66.936) (width 0.4) (layer B.Cu) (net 6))
 (segment (start 32.385 67.5132) (end 33.535 67.5132) (width 0.4) (layer B.Cu) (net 6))
 (segment (start 34.1122 65.3706) (end 35.5256 63.9572) (width 0.4) (layer B.Cu) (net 6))
 (segment (start 34.1122 66.936) (end 34.1122 65.3706) (width 0.4) (layer B.Cu) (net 6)))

